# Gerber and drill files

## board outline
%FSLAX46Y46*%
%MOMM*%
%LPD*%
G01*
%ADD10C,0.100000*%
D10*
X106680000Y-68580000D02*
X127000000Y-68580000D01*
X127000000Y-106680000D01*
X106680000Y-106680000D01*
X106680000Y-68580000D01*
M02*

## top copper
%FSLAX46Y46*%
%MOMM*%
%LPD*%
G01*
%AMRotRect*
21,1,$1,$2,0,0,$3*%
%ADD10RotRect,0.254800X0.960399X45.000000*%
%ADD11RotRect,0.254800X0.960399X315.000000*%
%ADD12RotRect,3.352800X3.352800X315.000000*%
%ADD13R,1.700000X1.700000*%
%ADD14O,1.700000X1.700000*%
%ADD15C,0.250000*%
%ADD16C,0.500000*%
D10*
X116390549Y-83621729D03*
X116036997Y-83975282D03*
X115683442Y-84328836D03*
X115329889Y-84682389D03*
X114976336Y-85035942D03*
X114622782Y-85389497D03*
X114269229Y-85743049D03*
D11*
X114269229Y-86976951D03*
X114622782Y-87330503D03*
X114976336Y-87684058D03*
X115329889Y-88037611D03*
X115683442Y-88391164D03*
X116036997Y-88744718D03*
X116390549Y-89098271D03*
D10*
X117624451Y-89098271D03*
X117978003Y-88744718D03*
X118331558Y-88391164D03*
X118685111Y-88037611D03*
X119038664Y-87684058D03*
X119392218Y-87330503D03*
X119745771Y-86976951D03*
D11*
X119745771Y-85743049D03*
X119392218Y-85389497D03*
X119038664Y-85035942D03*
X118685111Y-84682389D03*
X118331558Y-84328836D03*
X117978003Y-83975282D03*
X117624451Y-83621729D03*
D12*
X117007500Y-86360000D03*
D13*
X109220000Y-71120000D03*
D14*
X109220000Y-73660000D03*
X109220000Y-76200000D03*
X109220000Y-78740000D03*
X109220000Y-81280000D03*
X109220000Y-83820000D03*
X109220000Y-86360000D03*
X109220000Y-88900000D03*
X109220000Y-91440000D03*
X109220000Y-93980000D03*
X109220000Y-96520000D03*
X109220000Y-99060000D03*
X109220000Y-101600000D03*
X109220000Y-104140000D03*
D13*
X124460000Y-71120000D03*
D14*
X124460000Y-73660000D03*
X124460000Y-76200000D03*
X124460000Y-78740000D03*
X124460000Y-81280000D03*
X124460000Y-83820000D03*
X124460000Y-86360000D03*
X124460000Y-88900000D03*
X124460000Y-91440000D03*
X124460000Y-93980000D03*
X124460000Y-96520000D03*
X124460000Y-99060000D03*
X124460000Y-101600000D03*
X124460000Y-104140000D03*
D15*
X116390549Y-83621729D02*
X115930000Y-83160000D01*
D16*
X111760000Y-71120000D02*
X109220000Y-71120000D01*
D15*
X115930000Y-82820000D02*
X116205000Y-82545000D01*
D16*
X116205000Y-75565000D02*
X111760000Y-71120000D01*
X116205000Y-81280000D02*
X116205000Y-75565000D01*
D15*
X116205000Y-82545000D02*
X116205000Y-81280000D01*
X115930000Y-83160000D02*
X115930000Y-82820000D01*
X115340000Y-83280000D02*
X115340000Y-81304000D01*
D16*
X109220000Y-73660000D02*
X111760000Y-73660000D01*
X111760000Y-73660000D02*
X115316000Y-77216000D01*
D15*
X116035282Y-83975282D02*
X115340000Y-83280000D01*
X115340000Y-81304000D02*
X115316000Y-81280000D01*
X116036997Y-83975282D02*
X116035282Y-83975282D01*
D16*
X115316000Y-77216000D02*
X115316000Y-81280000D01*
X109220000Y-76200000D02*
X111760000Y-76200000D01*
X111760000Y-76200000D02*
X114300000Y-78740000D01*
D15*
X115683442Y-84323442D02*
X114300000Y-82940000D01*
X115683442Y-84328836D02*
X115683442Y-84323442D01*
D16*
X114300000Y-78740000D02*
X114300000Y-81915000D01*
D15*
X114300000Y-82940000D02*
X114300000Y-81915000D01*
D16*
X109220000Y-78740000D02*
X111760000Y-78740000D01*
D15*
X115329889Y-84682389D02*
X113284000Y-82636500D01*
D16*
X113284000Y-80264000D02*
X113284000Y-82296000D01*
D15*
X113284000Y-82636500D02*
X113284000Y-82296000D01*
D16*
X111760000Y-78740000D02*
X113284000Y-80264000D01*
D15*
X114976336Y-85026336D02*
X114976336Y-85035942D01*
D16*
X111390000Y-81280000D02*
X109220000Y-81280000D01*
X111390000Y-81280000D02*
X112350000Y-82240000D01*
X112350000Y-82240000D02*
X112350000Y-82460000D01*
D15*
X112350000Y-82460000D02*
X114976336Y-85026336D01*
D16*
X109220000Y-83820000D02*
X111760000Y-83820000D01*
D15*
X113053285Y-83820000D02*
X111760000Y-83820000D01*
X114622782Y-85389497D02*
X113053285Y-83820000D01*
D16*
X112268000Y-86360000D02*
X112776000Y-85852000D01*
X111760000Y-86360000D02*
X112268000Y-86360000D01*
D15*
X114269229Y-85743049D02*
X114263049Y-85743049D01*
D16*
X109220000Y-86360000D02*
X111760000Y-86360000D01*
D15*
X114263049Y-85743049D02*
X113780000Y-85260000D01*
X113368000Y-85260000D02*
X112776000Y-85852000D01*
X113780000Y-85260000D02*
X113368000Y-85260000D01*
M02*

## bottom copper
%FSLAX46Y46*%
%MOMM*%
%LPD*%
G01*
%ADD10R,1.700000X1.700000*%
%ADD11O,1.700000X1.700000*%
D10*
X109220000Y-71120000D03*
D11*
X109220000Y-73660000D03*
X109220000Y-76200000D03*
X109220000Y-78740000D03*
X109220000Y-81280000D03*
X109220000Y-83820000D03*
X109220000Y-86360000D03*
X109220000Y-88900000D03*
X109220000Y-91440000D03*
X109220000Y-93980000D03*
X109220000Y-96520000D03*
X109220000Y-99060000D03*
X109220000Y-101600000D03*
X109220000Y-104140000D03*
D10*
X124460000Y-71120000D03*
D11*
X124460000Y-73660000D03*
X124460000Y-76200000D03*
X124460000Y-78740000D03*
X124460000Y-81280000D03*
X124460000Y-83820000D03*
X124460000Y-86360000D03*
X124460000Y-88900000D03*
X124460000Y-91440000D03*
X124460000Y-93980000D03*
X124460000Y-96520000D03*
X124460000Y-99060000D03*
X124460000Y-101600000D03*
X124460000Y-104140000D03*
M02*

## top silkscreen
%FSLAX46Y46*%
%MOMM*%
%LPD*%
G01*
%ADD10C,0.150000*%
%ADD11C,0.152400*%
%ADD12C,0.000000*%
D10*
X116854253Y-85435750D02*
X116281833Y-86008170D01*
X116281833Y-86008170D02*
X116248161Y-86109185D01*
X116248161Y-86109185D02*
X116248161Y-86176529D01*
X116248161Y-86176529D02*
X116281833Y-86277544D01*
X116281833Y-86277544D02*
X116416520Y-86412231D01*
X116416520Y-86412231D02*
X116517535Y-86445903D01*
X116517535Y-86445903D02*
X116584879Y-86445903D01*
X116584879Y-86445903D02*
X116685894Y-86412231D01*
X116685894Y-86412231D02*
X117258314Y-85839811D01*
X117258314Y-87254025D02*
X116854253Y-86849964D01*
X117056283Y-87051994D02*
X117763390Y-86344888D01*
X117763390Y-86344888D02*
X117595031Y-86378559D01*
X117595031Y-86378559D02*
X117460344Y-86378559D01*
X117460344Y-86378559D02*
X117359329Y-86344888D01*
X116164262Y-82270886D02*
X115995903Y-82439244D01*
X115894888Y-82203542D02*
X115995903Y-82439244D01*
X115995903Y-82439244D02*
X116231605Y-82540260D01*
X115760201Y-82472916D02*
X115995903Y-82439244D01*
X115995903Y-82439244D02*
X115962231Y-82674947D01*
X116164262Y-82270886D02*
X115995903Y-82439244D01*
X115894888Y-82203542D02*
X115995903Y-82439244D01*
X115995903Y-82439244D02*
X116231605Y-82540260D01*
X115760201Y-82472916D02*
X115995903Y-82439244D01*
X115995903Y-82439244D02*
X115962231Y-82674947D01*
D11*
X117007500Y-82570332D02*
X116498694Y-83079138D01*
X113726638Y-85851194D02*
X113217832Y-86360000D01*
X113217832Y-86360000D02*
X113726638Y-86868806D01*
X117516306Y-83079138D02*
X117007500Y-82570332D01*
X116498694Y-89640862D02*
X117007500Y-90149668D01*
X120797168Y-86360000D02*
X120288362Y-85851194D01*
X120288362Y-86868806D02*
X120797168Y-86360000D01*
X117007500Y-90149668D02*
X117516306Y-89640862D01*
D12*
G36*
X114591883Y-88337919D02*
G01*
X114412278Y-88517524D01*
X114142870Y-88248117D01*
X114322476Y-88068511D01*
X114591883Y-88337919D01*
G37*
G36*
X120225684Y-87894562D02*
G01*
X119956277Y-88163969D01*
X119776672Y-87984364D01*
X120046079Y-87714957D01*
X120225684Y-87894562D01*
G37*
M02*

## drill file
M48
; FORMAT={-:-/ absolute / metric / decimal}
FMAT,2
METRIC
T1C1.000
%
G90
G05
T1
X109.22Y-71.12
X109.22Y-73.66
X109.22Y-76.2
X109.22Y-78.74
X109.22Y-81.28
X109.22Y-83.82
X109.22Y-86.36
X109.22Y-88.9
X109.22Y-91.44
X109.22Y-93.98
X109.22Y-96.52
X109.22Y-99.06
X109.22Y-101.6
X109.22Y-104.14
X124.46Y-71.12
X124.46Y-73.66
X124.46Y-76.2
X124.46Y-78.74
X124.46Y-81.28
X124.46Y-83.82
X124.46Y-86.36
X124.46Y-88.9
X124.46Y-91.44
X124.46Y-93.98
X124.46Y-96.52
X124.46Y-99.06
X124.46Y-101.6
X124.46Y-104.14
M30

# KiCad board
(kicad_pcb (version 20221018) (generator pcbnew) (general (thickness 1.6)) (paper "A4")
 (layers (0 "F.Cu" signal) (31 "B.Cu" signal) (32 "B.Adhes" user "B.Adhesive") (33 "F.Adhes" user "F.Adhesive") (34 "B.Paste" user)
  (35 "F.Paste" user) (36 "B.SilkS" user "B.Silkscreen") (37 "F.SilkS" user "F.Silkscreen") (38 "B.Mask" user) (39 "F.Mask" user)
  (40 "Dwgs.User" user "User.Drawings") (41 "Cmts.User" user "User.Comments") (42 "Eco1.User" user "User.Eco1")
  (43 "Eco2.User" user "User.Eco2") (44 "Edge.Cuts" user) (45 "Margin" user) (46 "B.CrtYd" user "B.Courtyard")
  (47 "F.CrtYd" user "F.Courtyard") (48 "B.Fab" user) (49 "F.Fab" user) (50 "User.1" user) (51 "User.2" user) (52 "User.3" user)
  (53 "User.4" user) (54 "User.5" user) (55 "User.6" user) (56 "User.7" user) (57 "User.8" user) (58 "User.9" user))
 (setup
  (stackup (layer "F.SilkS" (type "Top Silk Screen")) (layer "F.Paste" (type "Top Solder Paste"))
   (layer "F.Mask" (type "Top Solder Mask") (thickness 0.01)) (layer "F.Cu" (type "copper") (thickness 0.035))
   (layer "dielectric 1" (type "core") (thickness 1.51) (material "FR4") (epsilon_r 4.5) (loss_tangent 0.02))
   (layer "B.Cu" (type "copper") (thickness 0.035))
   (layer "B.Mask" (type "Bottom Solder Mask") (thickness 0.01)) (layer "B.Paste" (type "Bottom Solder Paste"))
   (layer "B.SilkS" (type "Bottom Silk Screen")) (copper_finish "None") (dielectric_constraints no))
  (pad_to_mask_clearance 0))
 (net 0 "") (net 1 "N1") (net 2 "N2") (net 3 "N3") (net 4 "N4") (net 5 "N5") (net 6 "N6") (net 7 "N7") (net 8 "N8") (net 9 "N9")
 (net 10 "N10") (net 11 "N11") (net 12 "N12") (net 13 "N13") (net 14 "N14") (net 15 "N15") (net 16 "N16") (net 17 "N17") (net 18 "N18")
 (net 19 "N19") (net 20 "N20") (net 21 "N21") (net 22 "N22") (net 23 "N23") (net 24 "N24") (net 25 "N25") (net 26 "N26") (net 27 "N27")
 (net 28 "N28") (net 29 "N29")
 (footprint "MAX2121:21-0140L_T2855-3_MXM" (layer "F.Cu") (at 117.0075 86.36 -45)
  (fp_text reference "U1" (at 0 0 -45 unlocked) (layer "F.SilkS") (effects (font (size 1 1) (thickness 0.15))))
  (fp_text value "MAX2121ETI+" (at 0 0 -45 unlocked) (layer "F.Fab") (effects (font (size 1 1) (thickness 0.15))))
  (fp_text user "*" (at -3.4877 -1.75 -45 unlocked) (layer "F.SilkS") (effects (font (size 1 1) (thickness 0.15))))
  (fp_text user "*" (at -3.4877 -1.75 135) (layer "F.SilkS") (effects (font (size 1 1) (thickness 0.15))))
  (fp_line (start -2.6797 -2.6797) (end -2.6797 -1.96014) (stroke (width 0.1524) (type solid)) (layer "F.SilkS"))
  (fp_line (start -2.6797 1.96014) (end -2.6797 2.6797) (stroke (width 0.1524) (type solid)) (layer "F.SilkS"))
  (fp_line (start -2.6797 2.6797) (end -1.96014 2.6797) (stroke (width 0.1524) (type solid)) (layer "F.SilkS"))
  (fp_line (start -1.96014 -2.6797) (end -2.6797 -2.6797) (stroke (width 0.1524) (type solid)) (layer "F.SilkS"))
  (fp_line (start 1.96014 2.6797) (end 2.6797 2.6797) (stroke (width 0.1524) (type solid)) (layer "F.SilkS"))
  (fp_line (start 2.6797 -2.6797) (end 1.96014 -2.6797) (stroke (width 0.1524) (type solid)) (layer "F.SilkS"))
  (fp_line (start 2.6797 -1.96014) (end 2.6797 -2.6797) (stroke (width 0.1524) (type solid)) (layer "F.SilkS"))
  (fp_line (start 2.6797 2.6797) (end 2.6797 1.96014) (stroke (width 0.1524) (type solid)) (layer "F.SilkS"))
  (fp_poly
   (pts (xy -0.690499 3.106699) (xy -0.690499 3.360699) (xy -0.309499 3.360699) (xy -0.309499 3.106699)) (stroke (width 0) (type solid))
   (fill solid) (layer "F.SilkS"))
  (fp_poly
   (pts (xy 3.360699 -1.190501) (xy 3.360699 -0.809501) (xy 3.106699 -0.809501) (xy 3.106699 -1.190501)) (stroke (width 0) (type solid))
   (fill solid) (layer "F.SilkS"))
  (pad "1" smd rect (at -2.3725 -1.5 45) (size 0.2548 0.960399) (layers "F.Cu" "F.Paste" "F.Mask") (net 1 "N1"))
  (pad "2" smd rect (at -2.3725 -1.000001 45) (size 0.2548 0.960399) (layers "F.Cu" "F.Paste" "F.Mask") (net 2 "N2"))
  (pad "3" smd rect (at -2.3725 -0.499999 45) (size 0.2548 0.960399) (layers "F.Cu" "F.Paste" "F.Mask") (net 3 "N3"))
  (pad "4" smd rect (at -2.3725 0 45) (size 0.2548 0.960399) (layers "F.Cu" "F.Paste" "F.Mask") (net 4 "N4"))
  (pad "5" smd rect (at -2.3725 0.499999 45) (size 0.2548 0.960399) (layers "F.Cu" "F.Paste" "F.Mask") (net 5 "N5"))
  (pad "6" smd rect (at -2.3725 1.000001 45) (size 0.2548 0.960399) (layers "F.Cu" "F.Paste" "F.Mask") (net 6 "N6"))
  (pad "7" smd rect (at -2.3725 1.5 45) (size 0.2548 0.960399) (layers "F.Cu" "F.Paste" "F.Mask") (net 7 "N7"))
  (pad "8" smd rect (at -1.5 2.3725 315) (size 0.2548 0.960399) (layers "F.Cu" "F.Paste" "F.Mask") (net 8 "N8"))
  (pad "9" smd rect (at -1.000001 2.3725 315) (size 0.2548 0.960399) (layers "F.Cu" "F.Paste" "F.Mask") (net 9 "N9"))
  (pad "10" smd rect (at -0.499999 2.3725 315) (size 0.2548 0.960399) (layers "F.Cu" "F.Paste" "F.Mask") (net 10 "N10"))
  (pad "11" smd rect (at 0 2.3725 315) (size 0.2548 0.960399) (layers "F.Cu" "F.Paste" "F.Mask") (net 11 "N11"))
  (pad "12" smd rect (at 0.499999 2.3725 315) (size 0.2548 0.960399) (layers "F.Cu" "F.Paste" "F.Mask") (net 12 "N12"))
  (pad "13" smd rect (at 1.000001 2.3725 315) (size 0.2548 0.960399) (layers "F.Cu" "F.Paste" "F.Mask") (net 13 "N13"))
  (pad "14" smd rect (at 1.5 2.3725 315) (size 0.2548 0.960399) (layers "F.Cu" "F.Paste" "F.Mask") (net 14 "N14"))
  (pad "15" smd rect (at 2.3725 1.5 45) (size 0.2548 0.960399) (layers "F.Cu" "F.Paste" "F.Mask") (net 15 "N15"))
  (pad "16" smd rect (at 2.3725 1.000001 45) (size 0.2548 0.960399) (layers "F.Cu" "F.Paste" "F.Mask") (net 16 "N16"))
  (pad "17" smd rect (at 2.3725 0.499999 45) (size 0.2548 0.960399) (layers "F.Cu" "F.Paste" "F.Mask") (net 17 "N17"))
  (pad "18" smd rect (at 2.3725 0 45) (size 0.2548 0.960399) (layers "F.Cu" "F.Paste" "F.Mask") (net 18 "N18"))
  (pad "19" smd rect (at 2.3725 -0.499999 45) (size 0.2548 0.960399) (layers "F.Cu" "F.Paste" "F.Mask") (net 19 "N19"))
  (pad "20" smd rect (at 2.3725 -1.000001 45) (size 0.2548 0.960399) (layers "F.Cu" "F.Paste" "F.Mask") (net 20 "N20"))
  (pad "21" smd rect (at 2.3725 -1.5 45) (size 0.2548 0.960399) (layers "F.Cu" "F.Paste" "F.Mask") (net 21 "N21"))
  (pad "22" smd rect (at 1.5 -2.3725 315) (size 0.2548 0.960399) (layers "F.Cu" "F.Paste" "F.Mask") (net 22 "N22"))
  (pad "23" smd rect (at 1.000001 -2.3725 315) (size 0.2548 0.960399) (layers "F.Cu" "F.Paste" "F.Mask") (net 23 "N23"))
  (pad "24" smd rect (at 0.499999 -2.3725 315) (size 0.2548 0.960399) (layers "F.Cu" "F.Paste" "F.Mask") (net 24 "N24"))
  (pad "25" smd rect (at 0 -2.3725 315) (size 0.2548 0.960399) (layers "F.Cu" "F.Paste" "F.Mask") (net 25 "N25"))
  (pad "26" smd rect (at -0.499999 -2.3725 315) (size 0.2548 0.960399) (layers "F.Cu" "F.Paste" "F.Mask") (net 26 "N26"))
  (pad "27" smd rect (at -1.000001 -2.3725 315) (size 0.2548 0.960399) (layers "F.Cu" "F.Paste" "F.Mask") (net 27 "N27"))
  (pad "28" smd rect (at -1.5 -2.3725 315) (size 0.2548 0.960399) (layers "F.Cu" "F.Paste" "F.Mask") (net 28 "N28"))
  (pad "29" smd rect (at 0 0 315) (size 3.3528 3.3528) (layers "F.Cu" "F.Mask") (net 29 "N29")))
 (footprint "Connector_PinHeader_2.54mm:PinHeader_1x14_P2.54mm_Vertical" (layer "B.Cu") (at 109.22 71.12 180)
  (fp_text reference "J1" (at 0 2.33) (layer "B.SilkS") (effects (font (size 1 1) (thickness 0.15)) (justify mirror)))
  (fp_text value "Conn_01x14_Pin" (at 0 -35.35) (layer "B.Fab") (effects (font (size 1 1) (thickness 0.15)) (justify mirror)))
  (pad "1" thru_hole rect (at 0 0 180) (size 1.7 1.7) (drill 1) (layers "*.Cu" "*.Mask") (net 1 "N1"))
  (pad "2" thru_hole oval (at 0 -2.54 180) (size 1.7 1.7) (drill 1) (layers "*.Cu" "*.Mask") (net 2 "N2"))
  (pad "3" thru_hole oval (at 0 -5.08 180) (size 1.7 1.7) (drill 1) (layers "*.Cu" "*.Mask") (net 3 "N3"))
  (pad "4" thru_hole oval (at 0 -7.62 180) (size 1.7 1.7) (drill 1) (layers "*.Cu" "*.Mask") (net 4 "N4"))
  (pad "5" thru_hole oval (at 0 -10.16 180) (size 1.7 1.7) (drill 1) (layers "*.Cu" "*.Mask") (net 5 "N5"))
  (pad "6" thru_hole oval (at 0 -12.7 180) (size 1.7 1.7) (drill 1) (layers "*.Cu" "*.Mask") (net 6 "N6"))
  (pad "7" thru_hole oval (at 0 -15.24 180) (size 1.7 1.7) (drill 1) (layers "*.Cu" "*.Mask") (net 7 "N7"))
  (pad "8" thru_hole oval (at 0 -17.78 180) (size 1.7 1.7) (drill 1) (layers "*.Cu" "*.Mask") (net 8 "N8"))
  (pad "9" thru_hole oval (at 0 -20.32 180) (size 1.7 1.7) (drill 1) (layers "*.Cu" "*.Mask") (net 9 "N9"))
  (pad "10" thru_hole oval (at 0 -22.86 180) (size 1.7 1.7) (drill 1) (layers "*.Cu" "*.Mask") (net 10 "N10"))
  (pad "11" thru_hole oval (at 0 -25.4 180) (size 1.7 1.7) (drill 1) (layers "*.Cu" "*.Mask") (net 11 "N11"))
  (pad "12" thru_hole oval (at 0 -27.94 180) (size 1.7 1.7) (drill 1) (layers "*.Cu" "*.Mask") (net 12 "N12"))
  (pad "13" thru_hole oval (at 0 -30.48 180) (size 1.7 1.7) (drill 1) (layers "*.Cu" "*.Mask") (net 13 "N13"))
  (pad "14" thru_hole oval (at 0 -33.02 180) (size 1.7 1.7) (drill 1) (layers "*.Cu" "*.Mask") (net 14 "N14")))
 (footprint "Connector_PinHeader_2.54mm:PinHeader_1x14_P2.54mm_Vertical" (layer "B.Cu") (at 124.46 71.12 180)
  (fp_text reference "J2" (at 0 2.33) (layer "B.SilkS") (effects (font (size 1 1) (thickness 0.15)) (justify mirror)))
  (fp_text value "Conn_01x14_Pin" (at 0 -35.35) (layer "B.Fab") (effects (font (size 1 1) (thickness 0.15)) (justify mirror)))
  (pad "1" thru_hole rect (at 0 0 180) (size 1.7 1.7) (drill 1) (layers "*.Cu" "*.Mask") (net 28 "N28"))
  (pad "2" thru_hole oval (at 0 -2.54 180) (size 1.7 1.7) (drill 1) (layers "*.Cu" "*.Mask") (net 27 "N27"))
  (pad "3" thru_hole oval (at 0 -5.08 180) (size 1.7 1.7) (drill 1) (layers "*.Cu" "*.Mask") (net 26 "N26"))
  (pad "4" thru_hole oval (at 0 -7.62 180) (size 1.7 1.7) (drill 1) (layers "*.Cu" "*.Mask") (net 25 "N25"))
  (pad "5" thru_hole oval (at 0 -10.16 180) (size 1.7 1.7) (drill 1) (layers "*.Cu" "*.Mask") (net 24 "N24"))
  (pad "6" thru_hole oval (at 0 -12.7 180) (size 1.7 1.7) (drill 1) (layers "*.Cu" "*.Mask") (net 23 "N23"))
  (pad "7" thru_hole oval (at 0 -15.24 180) (size 1.7 1.7) (drill 1) (layers "*.Cu" "*.Mask") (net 22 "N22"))
  (pad "8" thru_hole oval (at 0 -17.78 180) (size 1.7 1.7) (drill 1) (layers "*.Cu" "*.Mask") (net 21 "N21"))
  (pad "9" thru_hole oval (at 0 -20.32 180) (size 1.7 1.7) (drill 1) (layers "*.Cu" "*.Mask") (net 20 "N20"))
  (pad "10" thru_hole oval (at 0 -22.86 180) (size 1.7 1.7) (drill 1) (layers "*.Cu" "*.Mask") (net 19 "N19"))
  (pad "11" thru_hole oval (at 0 -25.4 180) (size 1.7 1.7) (drill 1) (layers "*.Cu" "*.Mask") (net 18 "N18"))
  (pad "12" thru_hole oval (at 0 -27.94 180) (size 1.7 1.7) (drill 1) (layers "*.Cu" "*.Mask") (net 17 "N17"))
  (pad "13" thru_hole oval (at 0 -30.48 180) (size 1.7 1.7) (drill 1) (layers "*.Cu" "*.Mask") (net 16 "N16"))
  (pad "14" thru_hole oval (at 0 -33.02 180) (size 1.7 1.7) (drill 1) (layers "*.Cu" "*.Mask") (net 15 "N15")))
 (gr_rect (start 106.68 68.58) (end 127 106.68) (stroke (width 0.1) (type default)) (fill none) (layer "Edge.Cuts"))
 (segment (start 116.390549 83.621729) (end 115.93 83.16) (width 0.25) (layer "F.Cu") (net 1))
 (segment (start 111.76 71.12) (end 109.22 71.12) (width 0.5) (layer "F.Cu") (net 1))
 (segment (start 115.93 82.82) (end 116.205 82.545) (width 0.25) (layer "F.Cu") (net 1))
 (segment (start 116.205 75.565) (end 111.76 71.12) (width 0.5) (layer "F.Cu") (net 1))
 (segment (start 116.205 81.28) (end 116.205 75.565) (width 0.5) (layer "F.Cu") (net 1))
 (segment (start 116.205 82.545) (end 116.205 81.28) (width 0.25) (layer "F.Cu") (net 1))
 (segment (start 115.93 83.16) (end 115.93 82.82) (width 0.25) (layer "F.Cu") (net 1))
 (segment (start 115.34 83.28) (end 115.34 81.304) (width 0.25) (layer "F.Cu") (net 2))
 (segment (start 109.22 73.66) (end 111.76 73.66) (width 0.5) (layer "F.Cu") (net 2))
 (segment (start 111.76 73.66) (end 115.316 77.216) (width 0.5) (layer "F.Cu") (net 2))
 (segment (start 116.035282 83.975282) (end 115.34 83.28) (width 0.25) (layer "F.Cu") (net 2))
 (segment (start 115.34 81.304) (end 115.316 81.28) (width 0.25) (layer "F.Cu") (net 2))
 (segment (start 116.036997 83.975282) (end 116.035282 83.975282) (width 0.25) (layer "F.Cu") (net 2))
 (segment (start 115.316 77.216) (end 115.316 81.28) (width 0.5) (layer "F.Cu") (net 2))
 (segment (start 109.22 76.2) (end 111.76 76.2) (width 0.5) (layer "F.Cu") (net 3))
 (segment (start 111.76 76.2) (end 114.3 78.74) (width 0.5) (layer "F.Cu") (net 3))
 (segment (start 115.683442 84.323442) (end 114.3 82.94) (width 0.25) (layer "F.Cu") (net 3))
 (segment (start 115.683442 84.328836) (end 115.683442 84.323442) (width 0.25) (layer "F.Cu") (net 3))
 (segment (start 114.3 78.74) (end 114.3 81.915) (width 0.5) (layer "F.Cu") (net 3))
 (segment (start 114.3 82.94) (end 114.3 81.915) (width 0.25) (layer "F.Cu") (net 3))
 (segment (start 109.22 78.74) (end 111.76 78.74) (width 0.5) (layer "F.Cu") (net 4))
 (segment (start 115.329889 84.682389) (end 113.284 82.6365) (width 0.25) (layer "F.Cu") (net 4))
 (segment (start 113.284 80.264) (end 113.284 82.296) (width 0.5) (layer "F.Cu") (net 4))
 (segment (start 113.284 82.6365) (end 113.284 82.296) (width 0.25) (layer "F.Cu") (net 4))
 (segment (start 111.76 78.74) (end 113.284 80.264) (width 0.5) (layer "F.Cu") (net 4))
 (segment (start 114.976336 85.026336) (end 114.976336 85.035942) (width 0.25) (layer "F.Cu") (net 5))
 (segment (start 111.39 81.28) (end 109.22 81.28) (width 0.5) (layer "F.Cu") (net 5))
 (segment (start 111.39 81.28) (end 112.35 82.24) (width 0.5) (layer "F.Cu") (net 5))
 (segment (start 112.35 82.24) (end 112.35 82.46) (width 0.5) (layer "F.Cu") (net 5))
 (segment (start 112.35 82.46) (end 114.976336 85.026336) (width 0.25) (layer "F.Cu") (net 5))
 (segment (start 109.22 83.82) (end 111.76 83.82) (width 0.5) (layer "F.Cu") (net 6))
 (segment (start 113.053285 83.82) (end 111.76 83.82) (width 0.25) (layer "F.Cu") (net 6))
 (segment (start 114.622782 85.389497) (end 113.053285 83.82) (width 0.25) (layer "F.Cu") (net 6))
 (segment (start 112.268 86.36) (end 112.776 85.852) (width 0.5) (layer "F.Cu") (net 7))
 (segment (start 111.76 86.36) (end 112.268 86.36) (width 0.5) (layer "F.Cu") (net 7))
 (segment (start 114.269229 85.743049) (end 114.263049 85.743049) (width 0.25) (layer "F.Cu") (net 7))
 (segment (start 109.22 86.36) (end 111.76 86.36) (width 0.5) (layer "F.Cu") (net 7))
 (segment (start 114.263049 85.743049) (end 113.78 85.26) (width 0.25) (layer "F.Cu") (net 7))
 (segment (start 113.368 85.26) (end 112.776 85.852) (width 0.25) (layer "F.Cu") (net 7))
 (segment (start 113.78 85.26) (end 113.368 85.26) (width 0.25) (layer "F.Cu") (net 7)))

